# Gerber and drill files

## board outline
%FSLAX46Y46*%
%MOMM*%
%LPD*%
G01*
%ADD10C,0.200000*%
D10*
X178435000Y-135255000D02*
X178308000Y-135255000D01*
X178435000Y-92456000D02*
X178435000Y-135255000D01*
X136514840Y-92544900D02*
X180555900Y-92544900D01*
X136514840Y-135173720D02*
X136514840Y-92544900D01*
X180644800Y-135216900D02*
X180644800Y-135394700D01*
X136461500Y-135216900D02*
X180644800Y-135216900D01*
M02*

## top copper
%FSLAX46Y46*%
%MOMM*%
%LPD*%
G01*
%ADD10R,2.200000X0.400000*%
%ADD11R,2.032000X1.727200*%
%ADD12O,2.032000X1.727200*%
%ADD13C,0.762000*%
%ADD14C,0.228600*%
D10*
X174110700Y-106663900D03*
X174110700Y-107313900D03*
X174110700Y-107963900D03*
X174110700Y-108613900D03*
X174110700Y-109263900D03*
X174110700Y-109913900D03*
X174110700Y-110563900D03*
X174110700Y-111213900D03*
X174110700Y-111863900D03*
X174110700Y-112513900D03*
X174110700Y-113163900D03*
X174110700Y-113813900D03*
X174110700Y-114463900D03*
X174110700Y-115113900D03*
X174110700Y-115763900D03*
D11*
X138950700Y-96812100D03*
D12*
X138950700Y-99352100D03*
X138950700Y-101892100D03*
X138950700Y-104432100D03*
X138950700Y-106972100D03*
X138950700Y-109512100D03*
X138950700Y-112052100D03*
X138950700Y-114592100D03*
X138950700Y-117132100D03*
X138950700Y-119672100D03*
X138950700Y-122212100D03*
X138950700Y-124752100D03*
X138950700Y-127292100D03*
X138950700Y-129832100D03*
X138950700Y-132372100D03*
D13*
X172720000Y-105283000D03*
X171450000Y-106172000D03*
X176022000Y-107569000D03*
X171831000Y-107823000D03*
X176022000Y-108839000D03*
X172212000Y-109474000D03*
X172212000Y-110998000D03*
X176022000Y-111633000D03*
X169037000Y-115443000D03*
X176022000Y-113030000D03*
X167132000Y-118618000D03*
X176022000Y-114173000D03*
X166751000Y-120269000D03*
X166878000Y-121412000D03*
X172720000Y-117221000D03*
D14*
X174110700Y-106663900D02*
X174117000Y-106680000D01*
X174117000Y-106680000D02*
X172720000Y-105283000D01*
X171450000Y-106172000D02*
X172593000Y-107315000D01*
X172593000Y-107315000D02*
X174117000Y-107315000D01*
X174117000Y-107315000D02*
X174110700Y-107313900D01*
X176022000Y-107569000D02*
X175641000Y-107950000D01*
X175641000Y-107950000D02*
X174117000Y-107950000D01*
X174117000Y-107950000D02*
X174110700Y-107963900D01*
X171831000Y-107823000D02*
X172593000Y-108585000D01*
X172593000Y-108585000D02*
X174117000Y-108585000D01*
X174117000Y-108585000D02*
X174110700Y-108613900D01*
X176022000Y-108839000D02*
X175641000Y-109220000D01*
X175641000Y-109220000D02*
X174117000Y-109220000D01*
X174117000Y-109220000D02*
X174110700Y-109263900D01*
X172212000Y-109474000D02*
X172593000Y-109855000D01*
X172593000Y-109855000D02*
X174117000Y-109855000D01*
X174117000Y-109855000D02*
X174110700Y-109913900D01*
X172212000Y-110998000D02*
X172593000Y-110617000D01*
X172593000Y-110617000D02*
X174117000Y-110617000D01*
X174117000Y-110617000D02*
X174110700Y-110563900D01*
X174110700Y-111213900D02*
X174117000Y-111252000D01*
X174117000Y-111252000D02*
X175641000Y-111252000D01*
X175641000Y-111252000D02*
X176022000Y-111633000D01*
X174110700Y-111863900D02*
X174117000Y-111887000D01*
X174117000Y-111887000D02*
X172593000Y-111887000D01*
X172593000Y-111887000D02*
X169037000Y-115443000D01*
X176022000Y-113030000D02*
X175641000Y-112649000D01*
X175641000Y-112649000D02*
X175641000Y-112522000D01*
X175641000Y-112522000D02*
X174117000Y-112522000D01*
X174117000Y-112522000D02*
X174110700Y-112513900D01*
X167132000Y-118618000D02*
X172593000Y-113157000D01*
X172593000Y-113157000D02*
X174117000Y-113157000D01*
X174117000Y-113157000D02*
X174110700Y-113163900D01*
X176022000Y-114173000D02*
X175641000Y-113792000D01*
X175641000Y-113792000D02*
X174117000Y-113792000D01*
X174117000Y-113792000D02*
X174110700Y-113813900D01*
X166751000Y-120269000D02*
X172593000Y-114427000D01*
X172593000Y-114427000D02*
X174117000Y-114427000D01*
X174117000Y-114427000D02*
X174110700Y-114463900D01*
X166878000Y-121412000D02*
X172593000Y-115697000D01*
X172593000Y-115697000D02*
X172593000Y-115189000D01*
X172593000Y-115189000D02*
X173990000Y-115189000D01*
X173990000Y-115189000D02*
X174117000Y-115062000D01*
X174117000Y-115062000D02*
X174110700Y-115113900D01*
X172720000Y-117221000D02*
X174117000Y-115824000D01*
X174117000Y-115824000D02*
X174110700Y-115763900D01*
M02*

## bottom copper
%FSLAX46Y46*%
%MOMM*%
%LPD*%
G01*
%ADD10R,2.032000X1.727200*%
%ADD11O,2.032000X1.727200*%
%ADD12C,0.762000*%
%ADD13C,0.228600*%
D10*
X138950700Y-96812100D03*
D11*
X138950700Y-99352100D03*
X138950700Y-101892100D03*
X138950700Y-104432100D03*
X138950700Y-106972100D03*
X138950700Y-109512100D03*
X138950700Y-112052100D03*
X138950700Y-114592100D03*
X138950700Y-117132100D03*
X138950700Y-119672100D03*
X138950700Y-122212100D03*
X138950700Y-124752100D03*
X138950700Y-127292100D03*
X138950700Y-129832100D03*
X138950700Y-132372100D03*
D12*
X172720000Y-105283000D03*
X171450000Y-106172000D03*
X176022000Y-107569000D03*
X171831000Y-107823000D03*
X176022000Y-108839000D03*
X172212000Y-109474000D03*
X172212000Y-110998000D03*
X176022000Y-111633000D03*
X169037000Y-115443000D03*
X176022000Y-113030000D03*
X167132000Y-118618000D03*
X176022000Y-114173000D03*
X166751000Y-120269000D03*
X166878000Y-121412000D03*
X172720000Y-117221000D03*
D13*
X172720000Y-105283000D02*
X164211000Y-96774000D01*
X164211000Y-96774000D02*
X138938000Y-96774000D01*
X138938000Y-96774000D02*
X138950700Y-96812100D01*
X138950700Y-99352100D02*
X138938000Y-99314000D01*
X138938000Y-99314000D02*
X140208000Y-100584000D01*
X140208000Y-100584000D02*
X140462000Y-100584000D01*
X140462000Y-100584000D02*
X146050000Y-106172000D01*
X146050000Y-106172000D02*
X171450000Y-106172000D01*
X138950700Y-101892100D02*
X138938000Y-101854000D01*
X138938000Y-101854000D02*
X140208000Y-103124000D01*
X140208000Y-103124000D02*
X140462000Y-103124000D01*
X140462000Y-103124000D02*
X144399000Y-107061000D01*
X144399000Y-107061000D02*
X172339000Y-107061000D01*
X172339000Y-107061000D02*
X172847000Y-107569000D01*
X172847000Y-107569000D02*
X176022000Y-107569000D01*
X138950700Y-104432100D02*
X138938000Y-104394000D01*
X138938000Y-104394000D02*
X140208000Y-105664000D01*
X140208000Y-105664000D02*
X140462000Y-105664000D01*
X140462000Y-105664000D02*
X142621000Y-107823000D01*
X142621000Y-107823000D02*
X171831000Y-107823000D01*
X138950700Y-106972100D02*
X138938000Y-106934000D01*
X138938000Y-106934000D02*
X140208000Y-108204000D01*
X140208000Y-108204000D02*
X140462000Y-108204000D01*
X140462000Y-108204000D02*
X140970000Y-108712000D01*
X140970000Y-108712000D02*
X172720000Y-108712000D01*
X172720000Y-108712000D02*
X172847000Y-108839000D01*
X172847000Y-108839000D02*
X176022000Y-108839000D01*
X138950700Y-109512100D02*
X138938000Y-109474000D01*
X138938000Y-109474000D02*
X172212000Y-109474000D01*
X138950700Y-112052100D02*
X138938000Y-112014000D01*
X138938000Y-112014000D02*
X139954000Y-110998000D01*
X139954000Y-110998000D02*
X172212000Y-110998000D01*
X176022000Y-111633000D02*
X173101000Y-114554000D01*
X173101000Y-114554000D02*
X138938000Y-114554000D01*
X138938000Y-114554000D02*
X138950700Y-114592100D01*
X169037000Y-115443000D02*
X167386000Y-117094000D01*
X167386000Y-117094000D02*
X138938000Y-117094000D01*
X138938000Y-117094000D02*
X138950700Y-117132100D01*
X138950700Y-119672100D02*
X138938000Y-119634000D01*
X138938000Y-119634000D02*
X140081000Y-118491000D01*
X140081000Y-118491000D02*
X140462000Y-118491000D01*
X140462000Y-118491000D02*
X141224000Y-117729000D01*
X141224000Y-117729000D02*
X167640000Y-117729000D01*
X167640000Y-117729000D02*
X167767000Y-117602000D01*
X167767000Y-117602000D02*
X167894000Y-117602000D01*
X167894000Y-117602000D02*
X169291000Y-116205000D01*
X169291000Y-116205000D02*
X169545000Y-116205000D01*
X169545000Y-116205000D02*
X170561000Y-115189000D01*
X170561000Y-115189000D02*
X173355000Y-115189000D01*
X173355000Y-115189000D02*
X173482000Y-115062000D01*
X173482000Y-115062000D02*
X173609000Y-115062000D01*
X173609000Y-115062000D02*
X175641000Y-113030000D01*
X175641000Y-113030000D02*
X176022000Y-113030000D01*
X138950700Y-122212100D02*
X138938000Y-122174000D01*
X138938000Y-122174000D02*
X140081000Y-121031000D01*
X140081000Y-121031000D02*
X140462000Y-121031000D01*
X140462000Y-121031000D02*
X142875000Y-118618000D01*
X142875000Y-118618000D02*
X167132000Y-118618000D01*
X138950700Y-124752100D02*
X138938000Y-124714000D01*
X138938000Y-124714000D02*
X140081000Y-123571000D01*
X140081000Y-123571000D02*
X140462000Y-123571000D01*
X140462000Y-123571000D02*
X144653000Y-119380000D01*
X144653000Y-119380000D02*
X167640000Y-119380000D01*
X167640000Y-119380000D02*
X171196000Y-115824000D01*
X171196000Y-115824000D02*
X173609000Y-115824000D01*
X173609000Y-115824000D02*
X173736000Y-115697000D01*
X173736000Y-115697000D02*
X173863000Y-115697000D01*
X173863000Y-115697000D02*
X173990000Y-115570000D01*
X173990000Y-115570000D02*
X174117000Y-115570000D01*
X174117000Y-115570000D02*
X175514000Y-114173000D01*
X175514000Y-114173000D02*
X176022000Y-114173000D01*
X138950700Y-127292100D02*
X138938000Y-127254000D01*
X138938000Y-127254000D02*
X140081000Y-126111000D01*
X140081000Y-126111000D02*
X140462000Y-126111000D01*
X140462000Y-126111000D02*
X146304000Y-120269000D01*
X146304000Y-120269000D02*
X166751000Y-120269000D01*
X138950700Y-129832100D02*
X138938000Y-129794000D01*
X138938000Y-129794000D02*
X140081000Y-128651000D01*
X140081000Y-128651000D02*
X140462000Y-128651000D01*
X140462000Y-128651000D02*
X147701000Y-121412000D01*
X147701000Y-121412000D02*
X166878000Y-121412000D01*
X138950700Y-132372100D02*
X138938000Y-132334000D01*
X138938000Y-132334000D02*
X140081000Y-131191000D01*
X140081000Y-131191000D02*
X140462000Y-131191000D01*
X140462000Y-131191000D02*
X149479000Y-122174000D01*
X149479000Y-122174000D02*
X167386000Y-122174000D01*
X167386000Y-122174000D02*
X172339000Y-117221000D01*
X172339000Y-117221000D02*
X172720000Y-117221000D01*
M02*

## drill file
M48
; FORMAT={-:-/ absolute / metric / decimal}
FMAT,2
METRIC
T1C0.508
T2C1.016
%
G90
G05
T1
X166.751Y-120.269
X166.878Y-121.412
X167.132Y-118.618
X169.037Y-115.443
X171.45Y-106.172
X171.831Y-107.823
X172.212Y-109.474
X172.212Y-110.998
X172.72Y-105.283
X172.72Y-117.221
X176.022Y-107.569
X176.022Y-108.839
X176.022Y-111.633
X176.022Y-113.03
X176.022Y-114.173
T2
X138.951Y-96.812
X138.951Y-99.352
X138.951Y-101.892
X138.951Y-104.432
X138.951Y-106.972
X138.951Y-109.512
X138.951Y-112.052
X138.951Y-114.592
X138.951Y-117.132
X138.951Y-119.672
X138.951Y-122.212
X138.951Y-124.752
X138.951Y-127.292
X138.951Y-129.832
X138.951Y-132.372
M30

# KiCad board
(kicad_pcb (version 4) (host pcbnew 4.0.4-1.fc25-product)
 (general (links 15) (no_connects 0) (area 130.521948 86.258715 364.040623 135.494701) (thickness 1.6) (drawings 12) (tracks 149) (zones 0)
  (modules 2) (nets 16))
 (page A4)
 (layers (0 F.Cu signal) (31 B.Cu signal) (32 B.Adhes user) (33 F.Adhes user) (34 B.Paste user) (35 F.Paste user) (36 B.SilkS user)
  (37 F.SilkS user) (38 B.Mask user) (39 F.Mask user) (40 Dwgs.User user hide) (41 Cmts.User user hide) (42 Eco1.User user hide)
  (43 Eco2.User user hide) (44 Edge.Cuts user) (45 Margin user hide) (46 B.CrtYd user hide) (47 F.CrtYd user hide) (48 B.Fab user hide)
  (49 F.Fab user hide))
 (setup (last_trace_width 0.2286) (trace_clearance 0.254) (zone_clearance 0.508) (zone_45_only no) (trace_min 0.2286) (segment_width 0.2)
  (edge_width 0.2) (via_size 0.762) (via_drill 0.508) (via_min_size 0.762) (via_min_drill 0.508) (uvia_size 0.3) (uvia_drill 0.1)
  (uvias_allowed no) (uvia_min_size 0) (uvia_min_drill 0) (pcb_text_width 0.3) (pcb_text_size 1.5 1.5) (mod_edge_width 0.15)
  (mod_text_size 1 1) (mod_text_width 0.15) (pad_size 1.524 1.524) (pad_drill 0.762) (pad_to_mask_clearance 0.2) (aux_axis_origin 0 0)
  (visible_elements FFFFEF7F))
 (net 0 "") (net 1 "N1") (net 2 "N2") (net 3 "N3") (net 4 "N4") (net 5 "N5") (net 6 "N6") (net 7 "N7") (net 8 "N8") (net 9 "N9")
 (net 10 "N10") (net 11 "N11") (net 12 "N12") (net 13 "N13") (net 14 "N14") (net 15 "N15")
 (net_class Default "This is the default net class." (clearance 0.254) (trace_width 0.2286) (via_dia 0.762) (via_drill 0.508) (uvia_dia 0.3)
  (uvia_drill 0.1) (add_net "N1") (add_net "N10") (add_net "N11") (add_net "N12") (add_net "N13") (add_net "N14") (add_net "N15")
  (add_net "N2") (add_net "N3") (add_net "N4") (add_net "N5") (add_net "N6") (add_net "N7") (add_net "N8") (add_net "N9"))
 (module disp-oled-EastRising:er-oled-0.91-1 (layer F.Cu) (at 174.5107 111.2139 270)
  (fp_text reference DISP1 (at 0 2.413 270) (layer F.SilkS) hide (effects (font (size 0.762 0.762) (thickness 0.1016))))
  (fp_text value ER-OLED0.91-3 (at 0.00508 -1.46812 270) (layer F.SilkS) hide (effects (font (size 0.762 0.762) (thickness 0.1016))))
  (pad 1 smd rect (at -4.55 0.4 270) (size 0.4 2.2) (layers F.Cu F.Paste F.Mask) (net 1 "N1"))
  (pad 2 smd rect (at -3.9 0.4 270) (size 0.4 2.2) (layers F.Cu F.Paste F.Mask) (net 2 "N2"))
  (pad 3 smd rect (at -3.25 0.4 270) (size 0.4 2.2) (layers F.Cu F.Paste F.Mask) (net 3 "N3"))
  (pad 4 smd rect (at -2.6 0.4 270) (size 0.4 2.2) (layers F.Cu F.Paste F.Mask) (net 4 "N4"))
  (pad 5 smd rect (at -1.95 0.4 270) (size 0.4 2.2) (layers F.Cu F.Paste F.Mask) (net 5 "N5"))
  (pad 6 smd rect (at -1.3 0.4 270) (size 0.4 2.2) (layers F.Cu F.Paste F.Mask) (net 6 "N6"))
  (pad 7 smd rect (at -0.65 0.4 270) (size 0.4 2.2) (layers F.Cu F.Paste F.Mask) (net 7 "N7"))
  (pad 8 smd rect (at 0 0.4 270) (size 0.4 2.2) (layers F.Cu F.Paste F.Mask) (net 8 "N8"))
  (pad 9 smd rect (at 0.65 0.4 270) (size 0.4 2.2) (layers F.Cu F.Paste F.Mask) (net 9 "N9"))
  (pad 10 smd rect (at 1.3 0.4 270) (size 0.4 2.2) (layers F.Cu F.Paste F.Mask) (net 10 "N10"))
  (pad 11 smd rect (at 1.95 0.4 270) (size 0.4 2.2) (layers F.Cu F.Paste F.Mask) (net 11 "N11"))
  (pad 12 smd rect (at 2.6 0.4 270) (size 0.4 2.2) (layers F.Cu F.Paste F.Mask) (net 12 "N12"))
  (pad 13 smd rect (at 3.25 0.4 270) (size 0.4 2.2) (layers F.Cu F.Paste F.Mask) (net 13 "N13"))
  (pad 14 smd rect (at 3.9 0.4 270) (size 0.4 2.2) (layers F.Cu F.Paste F.Mask) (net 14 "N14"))
  (pad 15 smd rect (at 4.55 0.4 270) (size 0.4 2.2) (layers F.Cu F.Paste F.Mask) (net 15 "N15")))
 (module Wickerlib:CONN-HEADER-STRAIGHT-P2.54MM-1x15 (layer F.Cu) (at 138.9507 96.8121)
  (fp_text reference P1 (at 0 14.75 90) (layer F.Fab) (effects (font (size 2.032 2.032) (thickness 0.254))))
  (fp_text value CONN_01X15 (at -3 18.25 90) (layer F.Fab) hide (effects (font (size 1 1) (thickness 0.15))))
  (pad 1 thru_hole rect (at 0 0) (size 2.032 1.7272) (drill 1.016) (layers *.Cu *.Mask F.SilkS) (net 1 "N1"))
  (pad 2 thru_hole oval (at 0 2.54) (size 2.032 1.7272) (drill 1.016) (layers *.Cu *.Mask F.SilkS) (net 2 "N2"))
  (pad 3 thru_hole oval (at 0 5.08) (size 2.032 1.7272) (drill 1.016) (layers *.Cu *.Mask F.SilkS) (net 3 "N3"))
  (pad 4 thru_hole oval (at 0 7.62) (size 2.032 1.7272) (drill 1.016) (layers *.Cu *.Mask F.SilkS) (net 4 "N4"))
  (pad 5 thru_hole oval (at 0 10.16) (size 2.032 1.7272) (drill 1.016) (layers *.Cu *.Mask F.SilkS) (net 5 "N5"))
  (pad 6 thru_hole oval (at 0 12.7) (size 2.032 1.7272) (drill 1.016) (layers *.Cu *.Mask F.SilkS) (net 6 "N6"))
  (pad 7 thru_hole oval (at 0 15.24) (size 2.032 1.7272) (drill 1.016) (layers *.Cu *.Mask F.SilkS) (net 7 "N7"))
  (pad 8 thru_hole oval (at 0 17.78) (size 2.032 1.7272) (drill 1.016) (layers *.Cu *.Mask F.SilkS) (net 8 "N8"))
  (pad 9 thru_hole oval (at 0 20.32) (size 2.032 1.7272) (drill 1.016) (layers *.Cu *.Mask F.SilkS) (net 9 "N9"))
  (pad 10 thru_hole oval (at 0 22.86) (size 2.032 1.7272) (drill 1.016) (layers *.Cu *.Mask F.SilkS) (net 10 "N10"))
  (pad 11 thru_hole oval (at 0 25.4) (size 2.032 1.7272) (drill 1.016) (layers *.Cu *.Mask F.SilkS) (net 11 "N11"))
  (pad 12 thru_hole oval (at 0 27.94) (size 2.032 1.7272) (drill 1.016) (layers *.Cu *.Mask F.SilkS) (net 12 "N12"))
  (pad 13 thru_hole oval (at 0 30.48) (size 2.032 1.7272) (drill 1.016) (layers *.Cu *.Mask F.SilkS) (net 13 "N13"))
  (pad 14 thru_hole oval (at 0 33.02) (size 2.032 1.7272) (drill 1.016) (layers *.Cu *.Mask F.SilkS) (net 14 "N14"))
  (pad 15 thru_hole oval (at 0 35.56) (size 2.032 1.7272) (drill 1.016) (layers *.Cu *.Mask F.SilkS) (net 15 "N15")))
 (gr_line (start 178.435 135.255) (end 178.308 135.255) (angle 90) (layer Edge.Cuts) (width 0.2))
 (gr_line (start 178.435 92.456) (end 178.435 135.255) (angle 90) (layer Edge.Cuts) (width 0.2))
 (gr_line (start 136.51484 92.5449) (end 180.5559 92.5449) (angle 90) (layer Edge.Cuts) (width 0.2))
 (gr_line (start 136.51484 135.17372) (end 136.51484 92.5449) (angle 90) (layer Edge.Cuts) (width 0.2))
 (gr_line (start 180.6448 135.2169) (end 180.6448 135.3947) (angle 90) (layer Edge.Cuts) (width 0.2))
 (gr_line (start 136.4615 135.2169) (end 180.6448 135.2169) (angle 90) (layer Edge.Cuts) (width 0.2))
 (segment (start 174.1107 106.6639) (end 174.117 106.68) (width 0.2286) (layer F.Cu) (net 1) (status 80000))
 (segment (start 174.117 106.68) (end 172.72 105.283) (width 0.2286) (layer F.Cu) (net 1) (status 80000))
 (via (at 172.72 105.283) (size 0.762) (layers F.Cu B.Cu) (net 1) (status 80000))
 (segment (start 172.72 105.283) (end 164.211 96.774) (width 0.2286) (layer B.Cu) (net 1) (status 80000))
 (segment (start 164.211 96.774) (end 138.938 96.774) (width 0.2286) (layer B.Cu) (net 1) (status 80000))
 (segment (start 138.938 96.774) (end 138.9507 96.8121) (width 0.2286) (layer B.Cu) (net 1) (status 80000))
 (segment (start 138.9507 99.3521) (end 138.938 99.314) (width 0.2286) (layer B.Cu) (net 2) (status 80000))
 (segment (start 138.938 99.314) (end 140.208 100.584) (width 0.2286) (layer B.Cu) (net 2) (status 80000))
 (segment (start 140.208 100.584) (end 140.462 100.584) (width 0.2286) (layer B.Cu) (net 2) (status 80000))
 (segment (start 140.462 100.584) (end 146.05 106.172) (width 0.2286) (layer B.Cu) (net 2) (status 80000))
 (segment (start 146.05 106.172) (end 171.45 106.172) (width 0.2286) (layer B.Cu) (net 2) (status 80000))
 (via (at 171.45 106.172) (size 0.762) (layers F.Cu B.Cu) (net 2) (status 80000))
 (segment (start 171.45 106.172) (end 172.593 107.315) (width 0.2286) (layer F.Cu) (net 2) (status 80000))
 (segment (start 172.593 107.315) (end 174.117 107.315) (width 0.2286) (layer F.Cu) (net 2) (status 80000))
 (segment (start 174.117 107.315) (end 174.1107 107.3139) (width 0.2286) (layer F.Cu) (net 2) (status 80000))
 (segment (start 138.9507 101.8921) (end 138.938 101.854) (width 0.2286) (layer B.Cu) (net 3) (status 80000))
 (segment (start 138.938 101.854) (end 140.208 103.124) (width 0.2286) (layer B.Cu) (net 3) (status 80000))
 (segment (start 140.208 103.124) (end 140.462 103.124) (width 0.2286) (layer B.Cu) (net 3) (status 80000))
 (segment (start 140.462 103.124) (end 144.399 107.061) (width 0.2286) (layer B.Cu) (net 3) (status 80000))
 (segment (start 144.399 107.061) (end 172.339 107.061) (width 0.2286) (layer B.Cu) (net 3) (status 80000))
 (segment (start 172.339 107.061) (end 172.847 107.569) (width 0.2286) (layer B.Cu) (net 3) (status 80000))
 (segment (start 172.847 107.569) (end 176.022 107.569) (width 0.2286) (layer B.Cu) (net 3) (status 80000))
 (via (at 176.022 107.569) (size 0.762) (layers F.Cu B.Cu) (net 3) (status 80000))
 (segment (start 176.022 107.569) (end 175.641 107.95) (width 0.2286) (layer F.Cu) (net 3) (status 80000))
 (segment (start 175.641 107.95) (end 174.117 107.95) (width 0.2286) (layer F.Cu) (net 3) (status 80000))
 (segment (start 174.117 107.95) (end 174.1107 107.9639) (width 0.2286) (layer F.Cu) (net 3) (status 80000))
 (segment (start 138.9507 104.4321) (end 138.938 104.394) (width 0.2286) (layer B.Cu) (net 4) (status 80000))
 (segment (start 138.938 104.394) (end 140.208 105.664) (width 0.2286) (layer B.Cu) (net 4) (status 80000))
 (segment (start 140.208 105.664) (end 140.462 105.664) (width 0.2286) (layer B.Cu) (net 4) (status 80000))
 (segment (start 140.462 105.664) (end 142.621 107.823) (width 0.2286) (layer B.Cu) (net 4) (status 80000))
 (segment (start 142.621 107.823) (end 171.831 107.823) (width 0.2286) (layer B.Cu) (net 4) (status 80000))
 (via (at 171.831 107.823) (size 0.762) (layers F.Cu B.Cu) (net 4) (status 80000))
 (segment (start 171.831 107.823) (end 172.593 108.585) (width 0.2286) (layer F.Cu) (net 4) (status 80000))
 (segment (start 172.593 108.585) (end 174.117 108.585) (width 0.2286) (layer F.Cu) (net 4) (status 80000))
 (segment (start 174.117 108.585) (end 174.1107 108.6139) (width 0.2286) (layer F.Cu) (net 4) (status 80000))
 (segment (start 138.9507 106.9721) (end 138.938 106.934) (width 0.2286) (layer B.Cu) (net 5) (status 80000))
 (segment (start 138.938 106.934) (end 140.208 108.204) (width 0.2286) (layer B.Cu) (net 5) (status 80000))
 (segment (start 140.208 108.204) (end 140.462 108.204) (width 0.2286) (layer B.Cu) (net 5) (status 80000))
 (segment (start 140.462 108.204) (end 140.97 108.712) (width 0.2286) (layer B.Cu) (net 5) (status 80000))
 (segment (start 140.97 108.712) (end 172.72 108.712) (width 0.2286) (layer B.Cu) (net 5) (status 80000))
 (segment (start 172.72 108.712) (end 172.847 108.839) (width 0.2286) (layer B.Cu) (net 5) (status 80000))
 (segment (start 172.847 108.839) (end 176.022 108.839) (width 0.2286) (layer B.Cu) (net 5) (status 80000))
 (via (at 176.022 108.839) (size 0.762) (layers F.Cu B.Cu) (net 5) (status 80000))
 (segment (start 176.022 108.839) (end 175.641 109.22) (width 0.2286) (layer F.Cu) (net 5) (status 80000))
 (segment (start 175.641 109.22) (end 174.117 109.22) (width 0.2286) (layer F.Cu) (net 5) (status 80000))
 (segment (start 174.117 109.22) (end 174.1107 109.2639) (width 0.2286) (layer F.Cu) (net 5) (status 80000))
 (segment (start 138.9507 109.5121) (end 138.938 109.474) (width 0.2286) (layer B.Cu) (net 6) (status 80000))
 (segment (start 138.938 109.474) (end 172.212 109.474) (width 0.2286) (layer B.Cu) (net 6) (status 80000))
 (via (at 172.212 109.474) (size 0.762) (layers F.Cu B.Cu) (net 6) (status 80000))
 (segment (start 172.212 109.474) (end 172.593 109.855) (width 0.2286) (layer F.Cu) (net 6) (status 80000))
 (segment (start 172.593 109.855) (end 174.117 109.855) (width 0.2286) (layer F.Cu) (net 6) (status 80000))
 (segment (start 174.117 109.855) (end 174.1107 109.9139) (width 0.2286) (layer F.Cu) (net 6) (status 80000))
 (segment (start 138.9507 112.0521) (end 138.938 112.014) (width 0.2286) (layer B.Cu) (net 7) (status 80000))
 (segment (start 138.938 112.014) (end 139.954 110.998) (width 0.2286) (layer B.Cu) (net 7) (status 80000))
 (segment (start 139.954 110.998) (end 172.212 110.998) (width 0.2286) (layer B.Cu) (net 7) (status 80000))
 (via (at 172.212 110.998) (size 0.762) (layers F.Cu B.Cu) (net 7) (status 80000))
 (segment (start 172.212 110.998) (end 172.593 110.617) (width 0.2286) (layer F.Cu) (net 7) (status 80000))
 (segment (start 172.593 110.617) (end 174.117 110.617) (width 0.2286) (layer F.Cu) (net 7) (status 80000))
 (segment (start 174.117 110.617) (end 174.1107 110.5639) (width 0.2286) (layer F.Cu) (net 7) (status 80000))
 (segment (start 174.1107 111.2139) (end 174.117 111.252) (width 0.2286) (layer F.Cu) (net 8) (status 80000))
 (segment (start 174.117 111.252) (end 175.641 111.252) (width 0.2286) (layer F.Cu) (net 8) (status 80000))
 (segment (start 175.641 111.252) (end 176.022 111.633) (width 0.2286) (layer F.Cu) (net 8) (status 80000))
 (via (at 176.022 111.633) (size 0.762) (layers F.Cu B.Cu) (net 8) (status 80000))
 (segment (start 176.022 111.633) (end 173.101 114.554) (width 0.2286) (layer B.Cu) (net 8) (status 80000))
 (segment (start 173.101 114.554) (end 138.938 114.554) (width 0.2286) (layer B.Cu) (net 8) (status 80000))
 (segment (start 138.938 114.554) (end 138.9507 114.5921) (width 0.2286) (layer B.Cu) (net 8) (status 80000))
 (segment (start 174.1107 111.8639) (end 174.117 111.887) (width 0.2286) (layer F.Cu) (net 9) (status 80000))
 (segment (start 174.117 111.887) (end 172.593 111.887) (width 0.2286) (layer F.Cu) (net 9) (status 80000))
 (segment (start 172.593 111.887) (end 169.037 115.443) (width 0.2286) (layer F.Cu) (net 9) (status 80000))
 (via (at 169.037 115.443) (size 0.762) (layers F.Cu B.Cu) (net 9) (status 80000))
 (segment (start 169.037 115.443) (end 167.386 117.094) (width 0.2286) (layer B.Cu) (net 9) (status 80000))
 (segment (start 167.386 117.094) (end 138.938 117.094) (width 0.2286) (layer B.Cu) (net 9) (status 80000))
 (segment (start 138.938 117.094) (end 138.9507 117.1321) (width 0.2286) (layer B.Cu) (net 9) (status 80000))
 (segment (start 138.9507 119.6721) (end 138.938 119.634) (width 0.2286) (layer B.Cu) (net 10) (status 80000))
 (segment (start 138.938 119.634) (end 140.081 118.491) (width 0.2286) (layer B.Cu) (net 10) (status 80000))
 (segment (start 140.081 118.491) (end 140.462 118.491) (width 0.2286) (layer B.Cu) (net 10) (status 80000))
 (segment (start 140.462 118.491) (end 141.224 117.729) (width 0.2286) (layer B.Cu) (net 10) (status 80000))
 (segment (start 141.224 117.729) (end 167.64 117.729) (width 0.2286) (layer B.Cu) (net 10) (status 80000))
 (segment (start 167.64 117.729) (end 167.767 117.602) (width 0.2286) (layer B.Cu) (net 10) (status 80000))
 (segment (start 167.767 117.602) (end 167.894 117.602) (width 0.2286) (layer B.Cu) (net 10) (status 80000))
 (segment (start 167.894 117.602) (end 169.291 116.205) (width 0.2286) (layer B.Cu) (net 10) (status 80000))
 (segment (start 169.291 116.205) (end 169.545 116.205) (width 0.2286) (layer B.Cu) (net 10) (status 80000))
 (segment (start 169.545 116.205) (end 170.561 115.189) (width 0.2286) (layer B.Cu) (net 10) (status 80000))
 (segment (start 170.561 115.189) (end 173.355 115.189) (width 0.2286) (layer B.Cu) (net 10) (status 80000))
 (segment (start 173.355 115.189) (end 173.482 115.062) (width 0.2286) (layer B.Cu) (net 10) (status 80000))
 (segment (start 173.482 115.062) (end 173.609 115.062) (width 0.2286) (layer B.Cu) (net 10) (status 80000))
 (segment (start 173.609 115.062) (end 175.641 113.03) (width 0.2286) (layer B.Cu) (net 10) (status 80000))
 (segment (start 175.641 113.03) (end 176.022 113.03) (width 0.2286) (layer B.Cu) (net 10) (status 80000))
 (via (at 176.022 113.03) (size 0.762) (layers F.Cu B.Cu) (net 10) (status 80000))
 (segment (start 176.022 113.03) (end 175.641 112.649) (width 0.2286) (layer F.Cu) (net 10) (status 80000))
 (segment (start 175.641 112.649) (end 175.641 112.522) (width 0.2286) (layer F.Cu) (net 10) (status 80000))
 (segment (start 175.641 112.522) (end 174.117 112.522) (width 0.2286) (layer F.Cu) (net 10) (status 80000))
 (segment (start 174.117 112.522) (end 174.1107 112.5139) (width 0.2286) (layer F.Cu) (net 10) (status 80000))
 (segment (start 138.9507 122.2121) (end 138.938 122.174) (width 0.2286) (layer B.Cu) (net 11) (status 80000))
 (segment (start 138.938 122.174) (end 140.081 121.031) (width 0.2286) (layer B.Cu) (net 11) (status 80000))
 (segment (start 140.081 121.031) (end 140.462 121.031) (width 0.2286) (layer B.Cu) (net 11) (status 80000))
 (segment (start 140.462 121.031) (end 142.875 118.618) (width 0.2286) (layer B.Cu) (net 11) (status 80000))
 (segment (start 142.875 118.618) (end 167.132 118.618) (width 0.2286) (layer B.Cu) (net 11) (status 80000))
 (via (at 167.132 118.618) (size 0.762) (layers F.Cu B.Cu) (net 11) (status 80000))
 (segment (start 167.132 118.618) (end 172.593 113.157) (width 0.2286) (layer F.Cu) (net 11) (status 80000))
 (segment (start 172.593 113.157) (end 174.117 113.157) (width 0.2286) (layer F.Cu) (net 11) (status 80000))
 (segment (start 174.117 113.157) (end 174.1107 113.1639) (width 0.2286) (layer F.Cu) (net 11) (status 80000))
 (segment (start 138.9507 124.7521) (end 138.938 124.714) (width 0.2286) (layer B.Cu) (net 12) (status 80000))
 (segment (start 138.938 124.714) (end 140.081 123.571) (width 0.2286) (layer B.Cu) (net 12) (status 80000))
 (segment (start 140.081 123.571) (end 140.462 123.571) (width 0.2286) (layer B.Cu) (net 12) (status 80000))
 (segment (start 140.462 123.571) (end 144.653 119.38) (width 0.2286) (layer B.Cu) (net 12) (status 80000))
 (segment (start 144.653 119.38) (end 167.64 119.38) (width 0.2286) (layer B.Cu) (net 12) (status 80000))
 (segment (start 167.64 119.38) (end 171.196 115.824) (width 0.2286) (layer B.Cu) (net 12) (status 80000))
 (segment (start 171.196 115.824) (end 173.609 115.824) (width 0.2286) (layer B.Cu) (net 12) (status 80000))
 (segment (start 173.609 115.824) (end 173.736 115.697) (width 0.2286) (layer B.Cu) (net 12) (status 80000))
 (segment (start 173.736 115.697) (end 173.863 115.697) (width 0.2286) (layer B.Cu) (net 12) (status 80000))
 (segment (start 173.863 115.697) (end 173.99 115.57) (width 0.2286) (layer B.Cu) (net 12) (status 80000))
 (segment (start 173.99 115.57) (end 174.117 115.57) (width 0.2286) (layer B.Cu) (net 12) (status 80000))
 (segment (start 174.117 115.57) (end 175.514 114.173) (width 0.2286) (layer B.Cu) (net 12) (status 80000))
 (segment (start 175.514 114.173) (end 176.022 114.173) (width 0.2286) (layer B.Cu) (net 12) (status 80000))
 (via (at 176.022 114.173) (size 0.762) (layers F.Cu B.Cu) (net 12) (status 80000))
 (segment (start 176.022 114.173) (end 175.641 113.792) (width 0.2286) (layer F.Cu) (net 12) (status 80000))
 (segment (start 175.641 113.792) (end 174.117 113.792) (width 0.2286) (layer F.Cu) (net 12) (status 80000))
 (segment (start 174.117 113.792) (end 174.1107 113.8139) (width 0.2286) (layer F.Cu) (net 12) (status 80000))
 (segment (start 138.9507 127.2921) (end 138.938 127.254) (width 0.2286) (layer B.Cu) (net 13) (status 80000))
 (segment (start 138.938 127.254) (end 140.081 126.111) (width 0.2286) (layer B.Cu) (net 13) (status 80000))
 (segment (start 140.081 126.111) (end 140.462 126.111) (width 0.2286) (layer B.Cu) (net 13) (status 80000))
 (segment (start 140.462 126.111) (end 146.304 120.269) (width 0.2286) (layer B.Cu) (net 13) (status 80000))
 (segment (start 146.304 120.269) (end 166.751 120.269) (width 0.2286) (layer B.Cu) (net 13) (status 80000))
 (via (at 166.751 120.269) (size 0.762) (layers F.Cu B.Cu) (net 13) (status 80000))
 (segment (start 166.751 120.269) (end 172.593 114.427) (width 0.2286) (layer F.Cu) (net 13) (status 80000))
 (segment (start 172.593 114.427) (end 174.117 114.427) (width 0.2286) (layer F.Cu) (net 13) (status 80000))
 (segment (start 174.117 114.427) (end 174.1107 114.4639) (width 0.2286) (layer F.Cu) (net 13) (status 80000))
 (segment (start 138.9507 129.8321) (end 138.938 129.794) (width 0.2286) (layer B.Cu) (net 14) (status 80000))
 (segment (start 138.938 129.794) (end 140.081 128.651) (width 0.2286) (layer B.Cu) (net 14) (status 80000))
 (segment (start 140.081 128.651) (end 140.462 128.651) (width 0.2286) (layer B.Cu) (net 14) (status 80000))
 (segment (start 140.462 128.651) (end 147.701 121.412) (width 0.2286) (layer B.Cu) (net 14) (status 80000))
 (segment (start 147.701 121.412) (end 166.878 121.412) (width 0.2286) (layer B.Cu) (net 14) (status 80000))
 (via (at 166.878 121.412) (size 0.762) (layers F.Cu B.Cu) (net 14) (status 80000))
 (segment (start 166.878 121.412) (end 172.593 115.697) (width 0.2286) (layer F.Cu) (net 14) (status 80000))
 (segment (start 172.593 115.697) (end 172.593 115.189) (width 0.2286) (layer F.Cu) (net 14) (status 80000))
 (segment (start 172.593 115.189) (end 173.99 115.189) (width 0.2286) (layer F.Cu) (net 14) (status 80000))
 (segment (start 173.99 115.189) (end 174.117 115.062) (width 0.2286) (layer F.Cu) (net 14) (status 80000))
 (segment (start 174.117 115.062) (end 174.1107 115.1139) (width 0.2286) (layer F.Cu) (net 14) (status 80000))
 (segment (start 138.9507 132.3721) (end 138.938 132.334) (width 0.2286) (layer B.Cu) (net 15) (status 80000))
 (segment (start 138.938 132.334) (end 140.081 131.191) (width 0.2286) (layer B.Cu) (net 15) (status 80000))
 (segment (start 140.081 131.191) (end 140.462 131.191) (width 0.2286) (layer B.Cu) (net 15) (status 80000))
 (segment (start 140.462 131.191) (end 149.479 122.174) (width 0.2286) (layer B.Cu) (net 15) (status 80000))
 (segment (start 149.479 122.174) (end 167.386 122.174) (width 0.2286) (layer B.Cu) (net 15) (status 80000))
 (segment (start 167.386 122.174) (end 172.339 117.221) (width 0.2286) (layer B.Cu) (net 15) (status 80000))
 (segment (start 172.339 117.221) (end 172.72 117.221) (width 0.2286) (layer B.Cu) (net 15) (status 80000))
 (via (at 172.72 117.221) (size 0.762) (layers F.Cu B.Cu) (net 15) (status 80000))
 (segment (start 172.72 117.221) (end 174.117 115.824) (width 0.2286) (layer F.Cu) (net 15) (status 80000))
 (segment (start 174.117 115.824) (end 174.1107 115.7639) (width 0.2286) (layer F.Cu) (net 15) (status 80000)))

